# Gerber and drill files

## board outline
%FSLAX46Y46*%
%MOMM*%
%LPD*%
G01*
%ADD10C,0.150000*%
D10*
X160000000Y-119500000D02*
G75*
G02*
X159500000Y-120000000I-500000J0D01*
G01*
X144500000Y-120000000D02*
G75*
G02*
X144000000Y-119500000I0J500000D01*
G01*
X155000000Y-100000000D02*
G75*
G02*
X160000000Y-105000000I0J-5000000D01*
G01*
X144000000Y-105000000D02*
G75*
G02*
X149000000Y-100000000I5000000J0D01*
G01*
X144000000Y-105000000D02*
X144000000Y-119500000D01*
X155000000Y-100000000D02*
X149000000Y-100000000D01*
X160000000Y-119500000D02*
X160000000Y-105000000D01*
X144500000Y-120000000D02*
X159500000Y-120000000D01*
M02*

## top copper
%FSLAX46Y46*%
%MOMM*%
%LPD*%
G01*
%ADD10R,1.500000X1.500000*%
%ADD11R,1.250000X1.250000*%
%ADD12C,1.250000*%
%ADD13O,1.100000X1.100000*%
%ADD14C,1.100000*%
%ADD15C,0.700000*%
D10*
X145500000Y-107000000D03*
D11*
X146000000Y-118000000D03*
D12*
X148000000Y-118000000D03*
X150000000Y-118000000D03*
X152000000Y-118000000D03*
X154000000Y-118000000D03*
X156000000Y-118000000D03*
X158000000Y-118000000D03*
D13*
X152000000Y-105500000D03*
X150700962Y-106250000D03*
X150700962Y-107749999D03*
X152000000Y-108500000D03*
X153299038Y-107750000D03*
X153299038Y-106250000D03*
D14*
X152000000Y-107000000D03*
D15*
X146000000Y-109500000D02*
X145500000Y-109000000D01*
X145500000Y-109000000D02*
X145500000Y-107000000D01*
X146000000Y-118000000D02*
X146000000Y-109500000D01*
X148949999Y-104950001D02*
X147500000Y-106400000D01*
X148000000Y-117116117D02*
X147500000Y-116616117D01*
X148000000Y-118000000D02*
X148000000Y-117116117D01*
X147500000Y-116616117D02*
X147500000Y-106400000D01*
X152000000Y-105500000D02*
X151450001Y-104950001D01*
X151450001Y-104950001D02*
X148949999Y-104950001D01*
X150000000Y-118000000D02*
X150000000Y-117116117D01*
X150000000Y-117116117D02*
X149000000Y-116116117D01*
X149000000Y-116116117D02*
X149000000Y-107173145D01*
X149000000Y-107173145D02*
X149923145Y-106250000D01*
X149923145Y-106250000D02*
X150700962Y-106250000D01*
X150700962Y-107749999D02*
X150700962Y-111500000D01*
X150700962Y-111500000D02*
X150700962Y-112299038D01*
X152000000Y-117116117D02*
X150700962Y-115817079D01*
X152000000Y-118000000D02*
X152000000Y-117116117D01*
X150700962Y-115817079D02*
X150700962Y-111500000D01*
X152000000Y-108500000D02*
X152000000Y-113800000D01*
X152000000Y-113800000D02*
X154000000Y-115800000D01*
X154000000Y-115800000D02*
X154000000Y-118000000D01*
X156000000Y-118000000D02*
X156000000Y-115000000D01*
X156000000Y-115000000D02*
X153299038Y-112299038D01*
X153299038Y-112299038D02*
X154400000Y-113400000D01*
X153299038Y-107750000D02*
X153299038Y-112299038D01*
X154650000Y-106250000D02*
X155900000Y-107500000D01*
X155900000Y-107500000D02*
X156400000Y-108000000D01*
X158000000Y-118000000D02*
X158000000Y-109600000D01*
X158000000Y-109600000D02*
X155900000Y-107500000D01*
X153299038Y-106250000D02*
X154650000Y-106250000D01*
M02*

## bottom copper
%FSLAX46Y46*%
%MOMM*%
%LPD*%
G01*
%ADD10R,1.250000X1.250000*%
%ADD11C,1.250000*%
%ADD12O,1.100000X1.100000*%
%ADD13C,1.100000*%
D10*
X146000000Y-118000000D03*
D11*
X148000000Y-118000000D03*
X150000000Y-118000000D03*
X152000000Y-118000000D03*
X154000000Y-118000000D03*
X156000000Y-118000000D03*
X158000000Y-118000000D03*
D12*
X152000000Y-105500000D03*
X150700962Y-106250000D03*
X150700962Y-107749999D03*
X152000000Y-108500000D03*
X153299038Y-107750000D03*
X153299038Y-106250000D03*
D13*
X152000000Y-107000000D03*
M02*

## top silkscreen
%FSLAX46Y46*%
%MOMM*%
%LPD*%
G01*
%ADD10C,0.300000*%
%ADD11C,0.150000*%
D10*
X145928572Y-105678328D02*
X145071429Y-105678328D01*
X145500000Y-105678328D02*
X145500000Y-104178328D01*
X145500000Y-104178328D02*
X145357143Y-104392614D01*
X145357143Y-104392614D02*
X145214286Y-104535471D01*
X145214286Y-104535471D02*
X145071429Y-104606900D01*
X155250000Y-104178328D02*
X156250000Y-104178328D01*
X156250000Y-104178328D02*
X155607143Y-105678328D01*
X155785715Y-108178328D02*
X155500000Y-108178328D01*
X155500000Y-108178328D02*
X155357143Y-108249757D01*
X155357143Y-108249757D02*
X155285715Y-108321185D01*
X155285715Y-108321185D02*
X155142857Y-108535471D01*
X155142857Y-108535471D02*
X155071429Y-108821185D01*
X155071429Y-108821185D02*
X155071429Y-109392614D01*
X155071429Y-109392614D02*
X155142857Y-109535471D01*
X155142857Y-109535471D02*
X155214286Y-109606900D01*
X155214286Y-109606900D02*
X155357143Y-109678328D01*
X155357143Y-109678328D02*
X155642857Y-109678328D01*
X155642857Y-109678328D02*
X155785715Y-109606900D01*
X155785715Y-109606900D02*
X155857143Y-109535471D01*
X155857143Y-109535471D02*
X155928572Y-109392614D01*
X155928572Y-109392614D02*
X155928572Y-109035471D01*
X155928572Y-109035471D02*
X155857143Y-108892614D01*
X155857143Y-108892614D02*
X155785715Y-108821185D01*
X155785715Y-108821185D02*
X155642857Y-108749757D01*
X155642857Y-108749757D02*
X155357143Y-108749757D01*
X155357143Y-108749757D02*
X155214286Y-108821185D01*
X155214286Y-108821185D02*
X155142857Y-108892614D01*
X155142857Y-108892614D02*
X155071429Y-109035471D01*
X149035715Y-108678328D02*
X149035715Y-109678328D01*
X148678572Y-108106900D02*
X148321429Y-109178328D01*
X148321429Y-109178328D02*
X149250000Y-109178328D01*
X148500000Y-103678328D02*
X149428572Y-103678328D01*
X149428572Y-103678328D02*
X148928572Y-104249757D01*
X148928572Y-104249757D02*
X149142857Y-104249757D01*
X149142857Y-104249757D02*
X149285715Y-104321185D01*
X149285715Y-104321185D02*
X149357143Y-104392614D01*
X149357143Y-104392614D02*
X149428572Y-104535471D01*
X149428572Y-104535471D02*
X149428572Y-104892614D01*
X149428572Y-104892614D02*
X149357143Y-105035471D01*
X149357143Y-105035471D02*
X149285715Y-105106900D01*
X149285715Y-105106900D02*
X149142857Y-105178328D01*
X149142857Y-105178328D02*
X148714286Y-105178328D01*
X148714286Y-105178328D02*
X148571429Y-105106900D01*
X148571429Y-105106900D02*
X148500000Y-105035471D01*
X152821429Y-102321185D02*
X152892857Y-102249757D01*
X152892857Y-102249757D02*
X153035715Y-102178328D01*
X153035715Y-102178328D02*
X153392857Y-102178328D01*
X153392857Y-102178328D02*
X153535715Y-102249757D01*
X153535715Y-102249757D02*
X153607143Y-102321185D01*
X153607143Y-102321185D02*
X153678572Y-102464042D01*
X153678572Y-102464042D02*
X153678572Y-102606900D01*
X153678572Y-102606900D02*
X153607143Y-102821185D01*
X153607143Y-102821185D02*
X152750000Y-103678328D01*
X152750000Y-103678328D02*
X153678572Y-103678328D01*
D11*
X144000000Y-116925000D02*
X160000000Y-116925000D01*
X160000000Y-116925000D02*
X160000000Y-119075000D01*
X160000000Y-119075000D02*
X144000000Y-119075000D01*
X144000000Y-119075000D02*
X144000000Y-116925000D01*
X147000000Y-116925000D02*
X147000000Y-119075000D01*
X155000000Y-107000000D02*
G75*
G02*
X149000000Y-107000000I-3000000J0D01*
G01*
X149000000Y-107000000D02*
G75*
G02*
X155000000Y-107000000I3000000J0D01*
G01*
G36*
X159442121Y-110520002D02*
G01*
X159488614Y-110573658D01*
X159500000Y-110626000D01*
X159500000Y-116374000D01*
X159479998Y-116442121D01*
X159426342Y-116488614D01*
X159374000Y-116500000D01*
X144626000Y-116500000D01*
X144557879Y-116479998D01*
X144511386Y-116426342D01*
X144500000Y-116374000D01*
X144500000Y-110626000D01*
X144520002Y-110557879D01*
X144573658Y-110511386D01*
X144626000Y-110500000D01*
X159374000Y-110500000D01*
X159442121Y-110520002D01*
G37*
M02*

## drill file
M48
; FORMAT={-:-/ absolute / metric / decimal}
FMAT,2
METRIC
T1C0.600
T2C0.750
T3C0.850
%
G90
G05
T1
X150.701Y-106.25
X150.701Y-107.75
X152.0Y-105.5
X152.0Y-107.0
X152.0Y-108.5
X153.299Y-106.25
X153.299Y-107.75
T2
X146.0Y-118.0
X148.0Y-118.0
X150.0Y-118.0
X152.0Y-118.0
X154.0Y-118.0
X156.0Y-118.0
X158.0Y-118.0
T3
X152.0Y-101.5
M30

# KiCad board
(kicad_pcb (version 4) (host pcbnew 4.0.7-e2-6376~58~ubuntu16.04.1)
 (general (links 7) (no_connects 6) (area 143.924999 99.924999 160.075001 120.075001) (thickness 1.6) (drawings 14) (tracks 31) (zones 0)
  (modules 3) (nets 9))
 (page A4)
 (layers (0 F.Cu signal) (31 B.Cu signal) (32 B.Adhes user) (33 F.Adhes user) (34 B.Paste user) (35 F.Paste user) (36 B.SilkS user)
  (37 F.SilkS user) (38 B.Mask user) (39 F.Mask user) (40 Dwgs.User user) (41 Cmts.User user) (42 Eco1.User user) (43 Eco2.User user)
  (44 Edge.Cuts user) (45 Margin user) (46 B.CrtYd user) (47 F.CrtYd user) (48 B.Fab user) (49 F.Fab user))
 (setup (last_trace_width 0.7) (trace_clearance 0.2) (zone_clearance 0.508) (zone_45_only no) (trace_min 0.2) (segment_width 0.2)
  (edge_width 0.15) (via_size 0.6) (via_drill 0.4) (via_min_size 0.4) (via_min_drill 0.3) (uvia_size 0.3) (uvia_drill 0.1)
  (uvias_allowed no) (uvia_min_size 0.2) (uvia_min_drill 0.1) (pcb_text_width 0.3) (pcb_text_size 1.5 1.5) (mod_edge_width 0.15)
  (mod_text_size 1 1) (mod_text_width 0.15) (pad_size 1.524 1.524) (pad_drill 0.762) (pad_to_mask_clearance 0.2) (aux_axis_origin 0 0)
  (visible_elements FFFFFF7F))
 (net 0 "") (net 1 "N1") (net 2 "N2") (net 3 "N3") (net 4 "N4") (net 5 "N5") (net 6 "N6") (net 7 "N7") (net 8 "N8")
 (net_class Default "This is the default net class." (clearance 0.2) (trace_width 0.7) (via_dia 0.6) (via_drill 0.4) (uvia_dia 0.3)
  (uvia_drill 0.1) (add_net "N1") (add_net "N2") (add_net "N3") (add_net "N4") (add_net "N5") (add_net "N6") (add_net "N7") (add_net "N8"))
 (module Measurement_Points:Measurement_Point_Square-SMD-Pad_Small (layer F.Cu) (at 145.5 107)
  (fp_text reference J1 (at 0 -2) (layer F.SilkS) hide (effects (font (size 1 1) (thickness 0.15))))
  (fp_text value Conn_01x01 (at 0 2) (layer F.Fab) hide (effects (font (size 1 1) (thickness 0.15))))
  (pad 1 smd rect (at 0 0) (size 1.5 1.5) (layers F.Cu F.Mask) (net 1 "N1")))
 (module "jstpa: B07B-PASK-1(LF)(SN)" (layer F.Cu) (at 152 118)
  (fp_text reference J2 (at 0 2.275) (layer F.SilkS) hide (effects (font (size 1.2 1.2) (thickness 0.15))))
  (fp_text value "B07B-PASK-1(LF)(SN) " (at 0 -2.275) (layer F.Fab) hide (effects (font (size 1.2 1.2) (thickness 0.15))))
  (fp_line (start -8 -1.075) (end 8 -1.075) (layer F.SilkS) (width 0.15))
  (fp_line (start 8 -1.075) (end 8 1.075) (layer F.SilkS) (width 0.15))
  (fp_line (start 8 1.075) (end -8 1.075) (layer F.SilkS) (width 0.15))
  (fp_line (start -8 1.075) (end -8 -1.075) (layer F.SilkS) (width 0.15))
  (fp_line (start -5 -1.075) (end -5 1.075) (layer F.SilkS) (width 0.15))
  (pad 1 thru_hole rect (at -6 0) (size 1.25 1.25) (drill 0.75) (layers *.Cu *.Mask) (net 1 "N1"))
  (pad 2 thru_hole circle (at -4 0) (size 1.25 1.25) (drill 0.75) (layers *.Cu *.Mask) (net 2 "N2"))
  (pad 3 thru_hole circle (at -2 0) (size 1.25 1.25) (drill 0.75) (layers *.Cu *.Mask) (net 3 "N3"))
  (pad 4 thru_hole circle (at 0 0) (size 1.25 1.25) (drill 0.75) (layers *.Cu *.Mask) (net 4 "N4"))
  (pad 5 thru_hole circle (at 2 0) (size 1.25 1.25) (drill 0.75) (layers *.Cu *.Mask) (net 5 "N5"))
  (pad 6 thru_hole circle (at 4 0) (size 1.25 1.25) (drill 0.75) (layers *.Cu *.Mask) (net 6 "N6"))
  (pad 7 thru_hole circle (at 6 0) (size 1.25 1.25) (drill 0.75) (layers *.Cu *.Mask) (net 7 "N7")))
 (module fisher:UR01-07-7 (layer F.Cu) (at 152 107)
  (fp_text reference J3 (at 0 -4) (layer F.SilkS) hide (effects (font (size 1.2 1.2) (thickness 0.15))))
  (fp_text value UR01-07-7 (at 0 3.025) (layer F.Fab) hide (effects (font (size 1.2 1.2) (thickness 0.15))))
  (fp_circle (center 0 0) (end 0 3) (layer F.SilkS) (width 0.15))
  (pad 2 thru_hole oval (at 0 -1.5) (size 1.1 1.1) (drill 0.6) (layers *.Cu *.Mask) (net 2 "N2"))
  (pad 3 thru_hole oval (at -1.299038 -0.75) (size 1.1 1.1) (drill 0.6) (layers *.Cu *.Mask) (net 3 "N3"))
  (pad 4 thru_hole oval (at -1.299038 0.749999) (size 1.1 1.1) (drill 0.6) (layers *.Cu *.Mask) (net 4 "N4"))
  (pad 5 thru_hole oval (at 0 1.5) (size 1.1 1.1) (drill 0.6) (layers *.Cu *.Mask) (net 5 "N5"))
  (pad 6 thru_hole oval (at 1.299038 0.75) (size 1.1 1.1) (drill 0.6) (layers *.Cu *.Mask) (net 6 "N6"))
  (pad 7 thru_hole oval (at 1.299038 -0.75) (size 1.1 1.1) (drill 0.6) (layers *.Cu *.Mask) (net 7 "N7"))
  (pad 1 thru_hole circle (at 0 0) (size 1.1 1.1) (drill 0.6) (layers *.Cu *.Mask) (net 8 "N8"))
  (pad "" np_thru_hole circle (at 0 -5.5) (size 0.85 0.85) (drill 0.85) (layers *.Cu *.Mask)))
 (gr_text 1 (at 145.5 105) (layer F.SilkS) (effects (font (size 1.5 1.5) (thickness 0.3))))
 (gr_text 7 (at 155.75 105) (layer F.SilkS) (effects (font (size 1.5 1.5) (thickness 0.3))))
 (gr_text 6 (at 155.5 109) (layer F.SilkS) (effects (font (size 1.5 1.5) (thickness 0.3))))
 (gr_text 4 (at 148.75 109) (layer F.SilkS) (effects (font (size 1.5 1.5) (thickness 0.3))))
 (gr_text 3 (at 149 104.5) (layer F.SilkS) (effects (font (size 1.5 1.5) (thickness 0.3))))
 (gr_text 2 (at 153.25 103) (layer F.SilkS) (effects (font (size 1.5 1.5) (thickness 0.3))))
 (gr_arc (start 159.5 119.5) (end 160 119.5) (angle 90) (layer Edge.Cuts) (width 0.15))
 (gr_arc (start 144.5 119.5) (end 144.5 120) (angle 90) (layer Edge.Cuts) (width 0.15))
 (gr_arc (start 155 105) (end 155 100) (angle 90) (layer Edge.Cuts) (width 0.15))
 (gr_arc (start 149 105) (end 144 105) (angle 90) (layer Edge.Cuts) (width 0.15))
 (gr_line (start 144 105) (end 144 119.5) (layer Edge.Cuts) (width 0.15))
 (gr_line (start 155 100) (end 149 100) (layer Edge.Cuts) (width 0.15))
 (gr_line (start 160 119.5) (end 160 105) (layer Edge.Cuts) (width 0.15))
 (gr_line (start 144.5 120) (end 159.5 120) (layer Edge.Cuts) (width 0.15))
 (segment (start 146 109.5) (end 145.5 109) (width 0.7) (layer F.Cu) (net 1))
 (segment (start 145.5 109) (end 145.5 107) (width 0.7) (layer F.Cu) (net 1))
 (segment (start 146 118) (end 146 109.5) (width 0.7) (layer F.Cu) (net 1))
 (segment (start 148.949999 104.950001) (end 147.5 106.4) (width 0.7) (layer F.Cu) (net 2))
 (segment (start 148 117.116117) (end 147.5 116.616117) (width 0.7) (layer F.Cu) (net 2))
 (segment (start 148 118) (end 148 117.116117) (width 0.7) (layer F.Cu) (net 2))
 (segment (start 147.5 116.616117) (end 147.5 106.4) (width 0.7) (layer F.Cu) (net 2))
 (segment (start 152 105.5) (end 151.450001 104.950001) (width 0.7) (layer F.Cu) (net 2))
 (segment (start 151.450001 104.950001) (end 148.949999 104.950001) (width 0.7) (layer F.Cu) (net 2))
 (segment (start 150 118) (end 150 117.116117) (width 0.7) (layer F.Cu) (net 3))
 (segment (start 150 117.116117) (end 149 116.116117) (width 0.7) (layer F.Cu) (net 3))
 (segment (start 149 116.116117) (end 149 107.173145) (width 0.7) (layer F.Cu) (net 3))
 (segment (start 149 107.173145) (end 149.923145 106.25) (width 0.7) (layer F.Cu) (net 3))
 (segment (start 149.923145 106.25) (end 150.700962 106.25) (width 0.7) (layer F.Cu) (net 3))
 (segment (start 150.700962 107.749999) (end 150.700962 111.5) (width 0.7) (layer F.Cu) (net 4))
 (segment (start 150.700962 111.5) (end 150.700962 112.299038) (width 0.7) (layer F.Cu) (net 4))
 (segment (start 152 117.116117) (end 150.700962 115.817079) (width 0.7) (layer F.Cu) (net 4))
 (segment (start 152 118) (end 152 117.116117) (width 0.7) (layer F.Cu) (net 4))
 (segment (start 150.700962 115.817079) (end 150.700962 111.5) (width 0.7) (layer F.Cu) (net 4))
 (segment (start 152 108.5) (end 152 113.8) (width 0.7) (layer F.Cu) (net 5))
 (segment (start 152 113.8) (end 154 115.8) (width 0.7) (layer F.Cu) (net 5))
 (segment (start 154 115.8) (end 154 118) (width 0.7) (layer F.Cu) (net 5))
 (segment (start 156 118) (end 156 115) (width 0.7) (layer F.Cu) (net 6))
 (segment (start 156 115) (end 153.299038 112.299038) (width 0.7) (layer F.Cu) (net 6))
 (segment (start 153.299038 112.299038) (end 154.4 113.4) (width 0.7) (layer F.Cu) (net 6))
 (segment (start 153.299038 107.75) (end 153.299038 112.299038) (width 0.7) (layer F.Cu) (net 6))
 (segment (start 154.65 106.25) (end 155.9 107.5) (width 0.7) (layer F.Cu) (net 7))
 (segment (start 155.9 107.5) (end 156.4 108) (width 0.7) (layer F.Cu) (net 7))
 (segment (start 158 118) (end 158 109.6) (width 0.7) (layer F.Cu) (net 7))
 (segment (start 158 109.6) (end 155.9 107.5) (width 0.7) (layer F.Cu) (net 7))
 (segment (start 153.299038 106.25) (end 154.65 106.25) (width 0.7) (layer F.Cu) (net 7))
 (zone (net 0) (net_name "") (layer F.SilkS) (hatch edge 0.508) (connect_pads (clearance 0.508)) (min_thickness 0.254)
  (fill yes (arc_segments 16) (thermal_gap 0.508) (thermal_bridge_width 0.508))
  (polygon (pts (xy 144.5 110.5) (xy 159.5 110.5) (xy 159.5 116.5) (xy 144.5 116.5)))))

